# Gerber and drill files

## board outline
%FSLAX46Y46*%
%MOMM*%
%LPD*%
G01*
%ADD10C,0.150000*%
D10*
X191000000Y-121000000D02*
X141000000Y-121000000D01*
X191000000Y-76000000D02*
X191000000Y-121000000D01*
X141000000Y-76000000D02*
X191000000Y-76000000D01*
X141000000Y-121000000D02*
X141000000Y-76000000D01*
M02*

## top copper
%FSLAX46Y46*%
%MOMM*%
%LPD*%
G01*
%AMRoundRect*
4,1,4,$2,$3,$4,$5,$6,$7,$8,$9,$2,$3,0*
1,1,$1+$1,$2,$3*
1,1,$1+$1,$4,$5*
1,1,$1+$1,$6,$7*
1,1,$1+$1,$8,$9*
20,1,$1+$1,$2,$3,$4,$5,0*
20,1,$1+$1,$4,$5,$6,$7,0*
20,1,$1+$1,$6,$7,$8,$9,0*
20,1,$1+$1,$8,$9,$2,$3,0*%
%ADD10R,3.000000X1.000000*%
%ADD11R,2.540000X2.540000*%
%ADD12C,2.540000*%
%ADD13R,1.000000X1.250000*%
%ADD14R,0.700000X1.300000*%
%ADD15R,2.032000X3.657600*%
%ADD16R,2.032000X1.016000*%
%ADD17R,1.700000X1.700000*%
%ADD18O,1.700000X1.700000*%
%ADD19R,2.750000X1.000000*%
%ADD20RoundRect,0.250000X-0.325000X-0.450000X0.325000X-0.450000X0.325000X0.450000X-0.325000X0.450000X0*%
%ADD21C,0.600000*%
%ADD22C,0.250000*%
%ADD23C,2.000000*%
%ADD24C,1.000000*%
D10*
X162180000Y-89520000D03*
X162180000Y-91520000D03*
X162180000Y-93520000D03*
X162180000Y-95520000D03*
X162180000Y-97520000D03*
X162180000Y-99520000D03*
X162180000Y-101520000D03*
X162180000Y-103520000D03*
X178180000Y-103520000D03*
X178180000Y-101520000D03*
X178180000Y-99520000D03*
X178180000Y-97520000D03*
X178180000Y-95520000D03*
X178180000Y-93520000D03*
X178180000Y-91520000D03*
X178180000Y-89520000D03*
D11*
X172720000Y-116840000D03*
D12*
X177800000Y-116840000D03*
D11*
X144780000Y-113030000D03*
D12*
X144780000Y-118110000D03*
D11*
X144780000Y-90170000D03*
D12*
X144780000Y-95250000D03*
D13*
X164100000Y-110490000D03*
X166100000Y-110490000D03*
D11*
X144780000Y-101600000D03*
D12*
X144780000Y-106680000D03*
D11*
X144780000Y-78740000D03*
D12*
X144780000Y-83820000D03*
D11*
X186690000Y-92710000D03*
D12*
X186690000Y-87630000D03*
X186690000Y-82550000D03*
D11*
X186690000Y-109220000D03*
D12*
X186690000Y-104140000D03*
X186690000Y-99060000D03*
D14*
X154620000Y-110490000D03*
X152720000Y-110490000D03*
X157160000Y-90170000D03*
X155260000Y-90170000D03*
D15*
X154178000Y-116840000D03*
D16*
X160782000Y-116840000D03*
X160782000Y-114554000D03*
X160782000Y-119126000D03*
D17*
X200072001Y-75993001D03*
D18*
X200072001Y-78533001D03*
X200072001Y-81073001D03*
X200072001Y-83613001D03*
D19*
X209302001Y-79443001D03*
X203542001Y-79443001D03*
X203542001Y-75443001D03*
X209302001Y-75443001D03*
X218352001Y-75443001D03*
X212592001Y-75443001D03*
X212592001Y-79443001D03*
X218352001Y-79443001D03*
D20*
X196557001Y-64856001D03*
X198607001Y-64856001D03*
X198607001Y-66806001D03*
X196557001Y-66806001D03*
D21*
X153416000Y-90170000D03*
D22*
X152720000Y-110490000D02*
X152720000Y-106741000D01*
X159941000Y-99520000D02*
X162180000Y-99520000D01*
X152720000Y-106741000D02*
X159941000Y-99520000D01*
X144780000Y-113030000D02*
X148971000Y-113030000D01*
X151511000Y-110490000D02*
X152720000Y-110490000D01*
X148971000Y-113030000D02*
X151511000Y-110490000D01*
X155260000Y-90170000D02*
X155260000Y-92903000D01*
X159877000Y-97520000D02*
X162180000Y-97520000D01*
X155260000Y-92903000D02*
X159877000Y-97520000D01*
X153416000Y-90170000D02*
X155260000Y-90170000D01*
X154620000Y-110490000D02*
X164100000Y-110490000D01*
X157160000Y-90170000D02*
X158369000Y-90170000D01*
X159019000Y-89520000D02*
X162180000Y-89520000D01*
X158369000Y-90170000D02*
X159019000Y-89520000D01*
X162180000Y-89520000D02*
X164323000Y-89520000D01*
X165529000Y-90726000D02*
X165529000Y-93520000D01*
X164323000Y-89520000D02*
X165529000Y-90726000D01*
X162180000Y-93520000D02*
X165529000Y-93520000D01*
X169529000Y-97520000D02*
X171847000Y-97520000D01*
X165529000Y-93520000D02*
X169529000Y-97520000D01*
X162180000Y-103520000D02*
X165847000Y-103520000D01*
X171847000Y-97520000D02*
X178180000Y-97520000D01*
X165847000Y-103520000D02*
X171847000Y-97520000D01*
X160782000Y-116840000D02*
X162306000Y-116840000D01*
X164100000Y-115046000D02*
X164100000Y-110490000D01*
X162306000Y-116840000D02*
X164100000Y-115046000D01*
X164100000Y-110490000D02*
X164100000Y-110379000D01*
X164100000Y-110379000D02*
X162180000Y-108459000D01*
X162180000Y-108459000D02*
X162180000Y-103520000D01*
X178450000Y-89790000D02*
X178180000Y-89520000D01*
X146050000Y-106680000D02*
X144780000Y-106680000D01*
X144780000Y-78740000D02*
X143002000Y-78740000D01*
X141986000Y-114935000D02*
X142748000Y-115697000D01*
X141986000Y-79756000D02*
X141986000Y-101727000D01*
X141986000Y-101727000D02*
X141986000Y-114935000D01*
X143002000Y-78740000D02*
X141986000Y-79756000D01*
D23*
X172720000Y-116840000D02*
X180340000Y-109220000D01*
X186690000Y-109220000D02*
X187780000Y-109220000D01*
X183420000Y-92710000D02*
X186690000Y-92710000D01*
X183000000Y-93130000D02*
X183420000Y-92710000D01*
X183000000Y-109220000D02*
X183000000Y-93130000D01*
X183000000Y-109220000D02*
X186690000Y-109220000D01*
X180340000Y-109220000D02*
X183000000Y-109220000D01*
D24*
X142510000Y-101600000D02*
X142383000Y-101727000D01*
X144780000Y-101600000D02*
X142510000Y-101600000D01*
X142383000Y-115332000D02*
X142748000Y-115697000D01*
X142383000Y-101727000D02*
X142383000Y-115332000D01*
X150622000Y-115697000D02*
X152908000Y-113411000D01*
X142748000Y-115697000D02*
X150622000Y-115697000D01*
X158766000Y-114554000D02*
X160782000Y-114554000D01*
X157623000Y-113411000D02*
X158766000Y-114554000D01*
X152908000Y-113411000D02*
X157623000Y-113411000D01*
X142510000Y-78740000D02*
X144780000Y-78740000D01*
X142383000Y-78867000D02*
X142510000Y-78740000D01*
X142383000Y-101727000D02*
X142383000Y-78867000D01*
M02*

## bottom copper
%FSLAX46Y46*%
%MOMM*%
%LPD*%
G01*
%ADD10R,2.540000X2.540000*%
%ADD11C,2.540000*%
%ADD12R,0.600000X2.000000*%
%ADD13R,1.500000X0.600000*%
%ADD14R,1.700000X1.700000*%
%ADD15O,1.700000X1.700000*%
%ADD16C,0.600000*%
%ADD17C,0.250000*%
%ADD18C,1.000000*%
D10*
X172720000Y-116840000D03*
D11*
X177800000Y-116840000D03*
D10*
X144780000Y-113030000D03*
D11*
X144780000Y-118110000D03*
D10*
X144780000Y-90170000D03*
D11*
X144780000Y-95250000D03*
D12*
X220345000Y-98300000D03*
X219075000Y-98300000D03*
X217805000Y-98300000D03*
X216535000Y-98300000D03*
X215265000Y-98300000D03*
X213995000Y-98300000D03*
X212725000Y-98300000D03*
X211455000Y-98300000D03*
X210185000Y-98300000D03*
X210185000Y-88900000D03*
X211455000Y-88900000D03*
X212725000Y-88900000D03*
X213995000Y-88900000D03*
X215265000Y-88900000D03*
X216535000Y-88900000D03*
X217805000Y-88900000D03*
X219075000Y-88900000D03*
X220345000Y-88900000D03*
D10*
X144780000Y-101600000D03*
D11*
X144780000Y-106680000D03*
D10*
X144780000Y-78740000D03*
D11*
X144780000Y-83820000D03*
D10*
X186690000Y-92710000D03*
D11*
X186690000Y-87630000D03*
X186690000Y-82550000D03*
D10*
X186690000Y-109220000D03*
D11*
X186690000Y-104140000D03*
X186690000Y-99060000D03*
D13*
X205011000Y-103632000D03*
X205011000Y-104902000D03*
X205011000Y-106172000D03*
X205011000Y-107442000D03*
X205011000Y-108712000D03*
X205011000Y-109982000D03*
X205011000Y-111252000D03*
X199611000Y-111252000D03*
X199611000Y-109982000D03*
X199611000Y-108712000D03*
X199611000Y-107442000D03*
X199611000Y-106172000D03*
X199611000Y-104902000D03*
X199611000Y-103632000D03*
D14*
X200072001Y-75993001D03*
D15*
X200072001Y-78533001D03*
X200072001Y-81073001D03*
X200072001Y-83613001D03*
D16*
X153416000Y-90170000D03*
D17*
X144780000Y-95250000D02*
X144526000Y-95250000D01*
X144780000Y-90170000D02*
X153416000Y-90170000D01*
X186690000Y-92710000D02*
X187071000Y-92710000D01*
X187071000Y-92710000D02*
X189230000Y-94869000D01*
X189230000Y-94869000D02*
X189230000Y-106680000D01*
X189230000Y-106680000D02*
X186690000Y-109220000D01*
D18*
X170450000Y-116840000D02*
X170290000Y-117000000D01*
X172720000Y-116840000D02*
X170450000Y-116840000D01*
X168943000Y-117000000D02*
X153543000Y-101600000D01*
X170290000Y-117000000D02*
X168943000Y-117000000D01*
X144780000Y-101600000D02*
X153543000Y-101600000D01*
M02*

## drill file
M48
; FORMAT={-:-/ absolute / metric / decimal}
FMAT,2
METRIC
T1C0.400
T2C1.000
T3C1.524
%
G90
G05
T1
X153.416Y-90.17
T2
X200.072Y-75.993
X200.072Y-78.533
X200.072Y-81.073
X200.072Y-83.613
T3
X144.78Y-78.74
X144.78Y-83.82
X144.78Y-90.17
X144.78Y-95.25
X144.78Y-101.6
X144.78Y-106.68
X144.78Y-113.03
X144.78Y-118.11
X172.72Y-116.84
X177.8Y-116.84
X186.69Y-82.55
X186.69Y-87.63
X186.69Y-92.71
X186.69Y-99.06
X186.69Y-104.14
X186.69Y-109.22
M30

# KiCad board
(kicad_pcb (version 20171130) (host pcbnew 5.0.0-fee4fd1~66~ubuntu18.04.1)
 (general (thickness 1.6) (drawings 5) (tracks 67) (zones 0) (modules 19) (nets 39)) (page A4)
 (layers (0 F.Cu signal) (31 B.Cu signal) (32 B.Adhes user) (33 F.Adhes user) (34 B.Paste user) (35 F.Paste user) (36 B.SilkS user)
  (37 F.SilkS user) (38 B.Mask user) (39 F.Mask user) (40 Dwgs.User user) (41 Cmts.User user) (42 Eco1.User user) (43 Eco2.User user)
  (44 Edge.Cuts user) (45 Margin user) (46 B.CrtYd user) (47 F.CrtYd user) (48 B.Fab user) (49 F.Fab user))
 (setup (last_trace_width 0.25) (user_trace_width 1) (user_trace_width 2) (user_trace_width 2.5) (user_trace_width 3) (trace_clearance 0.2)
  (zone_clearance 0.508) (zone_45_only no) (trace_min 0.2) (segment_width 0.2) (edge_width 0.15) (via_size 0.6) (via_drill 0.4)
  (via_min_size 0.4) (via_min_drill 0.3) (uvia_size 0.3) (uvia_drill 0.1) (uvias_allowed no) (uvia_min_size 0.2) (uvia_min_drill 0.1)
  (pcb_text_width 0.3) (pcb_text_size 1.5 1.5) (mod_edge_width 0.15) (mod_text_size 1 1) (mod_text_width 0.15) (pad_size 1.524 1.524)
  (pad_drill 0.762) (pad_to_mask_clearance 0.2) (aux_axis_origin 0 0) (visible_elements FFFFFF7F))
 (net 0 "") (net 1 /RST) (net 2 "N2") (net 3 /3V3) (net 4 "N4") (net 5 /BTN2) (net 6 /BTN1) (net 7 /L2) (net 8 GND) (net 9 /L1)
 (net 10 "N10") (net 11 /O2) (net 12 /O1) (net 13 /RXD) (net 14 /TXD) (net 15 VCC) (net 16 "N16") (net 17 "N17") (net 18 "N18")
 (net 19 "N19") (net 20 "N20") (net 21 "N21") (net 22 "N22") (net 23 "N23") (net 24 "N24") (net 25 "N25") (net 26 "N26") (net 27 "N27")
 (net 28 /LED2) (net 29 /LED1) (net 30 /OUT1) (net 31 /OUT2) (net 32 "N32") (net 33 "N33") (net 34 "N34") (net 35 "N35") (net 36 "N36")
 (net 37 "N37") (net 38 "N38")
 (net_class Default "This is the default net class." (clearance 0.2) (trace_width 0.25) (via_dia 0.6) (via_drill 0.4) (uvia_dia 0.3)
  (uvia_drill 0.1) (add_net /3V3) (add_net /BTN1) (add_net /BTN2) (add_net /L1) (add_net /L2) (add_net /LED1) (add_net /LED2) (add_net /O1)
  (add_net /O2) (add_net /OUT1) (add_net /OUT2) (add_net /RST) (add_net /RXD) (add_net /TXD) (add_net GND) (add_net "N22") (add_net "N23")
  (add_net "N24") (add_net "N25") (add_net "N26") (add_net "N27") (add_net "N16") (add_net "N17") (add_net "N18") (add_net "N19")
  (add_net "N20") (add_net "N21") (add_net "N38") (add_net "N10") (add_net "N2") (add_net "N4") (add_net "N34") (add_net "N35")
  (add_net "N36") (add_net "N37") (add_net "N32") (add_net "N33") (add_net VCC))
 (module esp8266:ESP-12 (layer F.Cu) (at 170.18 96.52)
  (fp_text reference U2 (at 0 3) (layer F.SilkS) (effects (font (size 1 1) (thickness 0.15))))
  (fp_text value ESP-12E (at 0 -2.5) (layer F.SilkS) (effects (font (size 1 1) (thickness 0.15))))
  (pad 1 smd rect (at -8 -7) (size 3 1) (layers F.Cu F.Paste F.Mask) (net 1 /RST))
  (pad 2 smd rect (at -8 -5) (size 3 1) (layers F.Cu F.Paste F.Mask) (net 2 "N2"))
  (pad 3 smd rect (at -8 -3) (size 3 1) (layers F.Cu F.Paste F.Mask) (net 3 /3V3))
  (pad 4 smd rect (at -8 -1) (size 3 1) (layers F.Cu F.Paste F.Mask) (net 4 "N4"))
  (pad 5 smd rect (at -8 1) (size 3 1) (layers F.Cu F.Paste F.Mask) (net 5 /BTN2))
  (pad 6 smd rect (at -8 3) (size 3 1) (layers F.Cu F.Paste F.Mask) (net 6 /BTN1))
  (pad 7 smd rect (at -8 5) (size 3 1) (layers F.Cu F.Paste F.Mask) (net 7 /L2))
  (pad 8 smd rect (at -8 7) (size 3 1) (layers F.Cu F.Paste F.Mask) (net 3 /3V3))
  (pad 9 smd rect (at 8 7) (size 3 1) (layers F.Cu F.Paste F.Mask) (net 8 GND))
  (pad 10 smd rect (at 8 5) (size 3 1) (layers F.Cu F.Paste F.Mask) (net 8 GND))
  (pad 11 smd rect (at 8 3) (size 3 1) (layers F.Cu F.Paste F.Mask) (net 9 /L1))
  (pad 12 smd rect (at 8 1) (size 3 1) (layers F.Cu F.Paste F.Mask) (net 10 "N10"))
  (pad 13 smd rect (at 8 -1) (size 3 1) (layers F.Cu F.Paste F.Mask) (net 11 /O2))
  (pad 14 smd rect (at 8 -3) (size 3 1) (layers F.Cu F.Paste F.Mask) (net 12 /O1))
  (pad 15 smd rect (at 8 -5) (size 3 1) (layers F.Cu F.Paste F.Mask) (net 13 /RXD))
  (pad 16 smd rect (at 8 -7) (size 3 1) (layers F.Cu F.Paste F.Mask) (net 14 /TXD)))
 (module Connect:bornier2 (layer F.Cu) (at 175.26 116.84)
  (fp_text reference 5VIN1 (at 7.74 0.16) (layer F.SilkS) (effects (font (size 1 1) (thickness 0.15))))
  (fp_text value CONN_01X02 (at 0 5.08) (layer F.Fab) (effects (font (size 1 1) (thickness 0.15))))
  (pad 1 thru_hole rect (at -2.54 0) (size 2.54 2.54) (drill 1.524) (layers *.Cu *.Mask F.SilkS) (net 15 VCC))
  (pad 2 thru_hole circle (at 2.54 0) (size 2.54 2.54) (drill 1.524) (layers *.Cu *.Mask F.SilkS) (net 8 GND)))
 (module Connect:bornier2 (layer F.Cu) (at 144.78 115.57 270)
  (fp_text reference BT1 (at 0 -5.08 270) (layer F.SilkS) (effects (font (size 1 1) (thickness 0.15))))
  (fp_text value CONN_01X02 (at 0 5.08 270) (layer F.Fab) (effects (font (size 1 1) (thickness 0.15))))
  (pad 1 thru_hole rect (at -2.54 0 270) (size 2.54 2.54) (drill 1.524) (layers *.Cu *.Mask F.SilkS) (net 6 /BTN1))
  (pad 2 thru_hole circle (at 2.54 0 270) (size 2.54 2.54) (drill 1.524) (layers *.Cu *.Mask F.SilkS) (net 8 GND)))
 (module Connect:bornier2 (layer F.Cu) (at 144.78 92.71 270)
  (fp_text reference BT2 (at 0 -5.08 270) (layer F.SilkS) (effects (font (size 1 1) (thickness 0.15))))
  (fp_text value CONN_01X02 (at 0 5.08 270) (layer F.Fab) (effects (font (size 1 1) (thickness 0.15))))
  (pad 1 thru_hole rect (at -2.54 0 270) (size 2.54 2.54) (drill 1.524) (layers *.Cu *.Mask F.SilkS) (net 5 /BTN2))
  (pad 2 thru_hole circle (at 2.54 0 270) (size 2.54 2.54) (drill 1.524) (layers *.Cu *.Mask F.SilkS) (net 8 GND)))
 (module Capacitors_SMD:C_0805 (layer F.Cu) (at 165.1 110.49)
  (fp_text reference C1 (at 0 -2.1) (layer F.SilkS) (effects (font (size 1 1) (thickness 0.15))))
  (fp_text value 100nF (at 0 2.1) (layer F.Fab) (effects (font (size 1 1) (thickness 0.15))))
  (pad 1 smd rect (at -1 0) (size 1 1.25) (layers F.Cu F.Paste F.Mask) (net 3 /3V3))
  (pad 2 smd rect (at 1 0) (size 1 1.25) (layers F.Cu F.Paste F.Mask) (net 8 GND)))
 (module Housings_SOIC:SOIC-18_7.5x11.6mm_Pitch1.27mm (layer B.Cu) (at 215.265 93.6 90)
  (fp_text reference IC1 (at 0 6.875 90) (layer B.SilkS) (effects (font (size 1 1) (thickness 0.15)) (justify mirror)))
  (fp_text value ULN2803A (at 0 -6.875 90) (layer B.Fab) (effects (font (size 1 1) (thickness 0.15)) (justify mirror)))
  (pad 1 smd rect (at -4.7 5.08 90) (size 2 0.6) (layers B.Cu B.Paste B.Mask) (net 9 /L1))
  (pad 2 smd rect (at -4.7 3.81 90) (size 2 0.6) (layers B.Cu B.Paste B.Mask) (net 7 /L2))
  (pad 3 smd rect (at -4.7 2.54 90) (size 2 0.6) (layers B.Cu B.Paste B.Mask) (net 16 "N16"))
  (pad 4 smd rect (at -4.7 1.27 90) (size 2 0.6) (layers B.Cu B.Paste B.Mask) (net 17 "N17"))
  (pad 5 smd rect (at -4.7 0 90) (size 2 0.6) (layers B.Cu B.Paste B.Mask) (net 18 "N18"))
  (pad 6 smd rect (at -4.7 -1.27 90) (size 2 0.6) (layers B.Cu B.Paste B.Mask) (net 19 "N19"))
  (pad 7 smd rect (at -4.7 -2.54 90) (size 2 0.6) (layers B.Cu B.Paste B.Mask) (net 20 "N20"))
  (pad 8 smd rect (at -4.7 -3.81 90) (size 2 0.6) (layers B.Cu B.Paste B.Mask) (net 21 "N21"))
  (pad 9 smd rect (at -4.7 -5.08 90) (size 2 0.6) (layers B.Cu B.Paste B.Mask) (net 8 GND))
  (pad 10 smd rect (at 4.7 -5.08 90) (size 2 0.6) (layers B.Cu B.Paste B.Mask) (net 15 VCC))
  (pad 11 smd rect (at 4.7 -3.81 90) (size 2 0.6) (layers B.Cu B.Paste B.Mask) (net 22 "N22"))
  (pad 12 smd rect (at 4.7 -2.54 90) (size 2 0.6) (layers B.Cu B.Paste B.Mask) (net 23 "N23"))
  (pad 13 smd rect (at 4.7 -1.27 90) (size 2 0.6) (layers B.Cu B.Paste B.Mask) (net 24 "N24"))
  (pad 14 smd rect (at 4.7 0 90) (size 2 0.6) (layers B.Cu B.Paste B.Mask) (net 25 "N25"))
  (pad 15 smd rect (at 4.7 1.27 90) (size 2 0.6) (layers B.Cu B.Paste B.Mask) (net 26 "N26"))
  (pad 16 smd rect (at 4.7 2.54 90) (size 2 0.6) (layers B.Cu B.Paste B.Mask) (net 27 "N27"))
  (pad 17 smd rect (at 4.7 3.81 90) (size 2 0.6) (layers B.Cu B.Paste B.Mask) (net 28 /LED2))
  (pad 18 smd rect (at 4.7 5.08 90) (size 2 0.6) (layers B.Cu B.Paste B.Mask) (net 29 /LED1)))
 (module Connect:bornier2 (layer F.Cu) (at 144.78 104.14 270)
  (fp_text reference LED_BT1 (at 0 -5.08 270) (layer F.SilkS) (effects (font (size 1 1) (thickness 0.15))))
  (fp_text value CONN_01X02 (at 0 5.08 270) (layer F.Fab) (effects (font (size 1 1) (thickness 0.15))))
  (pad 1 thru_hole rect (at -2.54 0 270) (size 2.54 2.54) (drill 1.524) (layers *.Cu *.Mask F.SilkS) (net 15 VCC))
  (pad 2 thru_hole circle (at 2.54 0 270) (size 2.54 2.54) (drill 1.524) (layers *.Cu *.Mask F.SilkS) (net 29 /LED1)))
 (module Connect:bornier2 (layer F.Cu) (at 144.78 81.28 270)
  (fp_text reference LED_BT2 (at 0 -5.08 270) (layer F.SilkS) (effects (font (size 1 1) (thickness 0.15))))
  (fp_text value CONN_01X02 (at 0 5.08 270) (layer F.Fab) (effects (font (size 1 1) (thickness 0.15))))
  (pad 1 thru_hole rect (at -2.54 0 270) (size 2.54 2.54) (drill 1.524) (layers *.Cu *.Mask F.SilkS) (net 15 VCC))
  (pad 2 thru_hole circle (at 2.54 0 270) (size 2.54 2.54) (drill 1.524) (layers *.Cu *.Mask F.SilkS) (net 28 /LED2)))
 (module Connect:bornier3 (layer F.Cu) (at 186.69 87.63 90)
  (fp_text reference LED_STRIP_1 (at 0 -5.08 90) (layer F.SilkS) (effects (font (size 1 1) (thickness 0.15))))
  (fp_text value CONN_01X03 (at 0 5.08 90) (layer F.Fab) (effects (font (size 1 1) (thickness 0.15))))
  (pad 1 thru_hole rect (at -5.08 0 90) (size 2.54 2.54) (drill 1.524) (layers *.Cu *.Mask F.SilkS) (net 15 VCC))
  (pad 2 thru_hole circle (at 0 0 90) (size 2.54 2.54) (drill 1.524) (layers *.Cu *.Mask F.SilkS) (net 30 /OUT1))
  (pad 3 thru_hole circle (at 5.08 0 90) (size 2.54 2.54) (drill 1.524) (layers *.Cu *.Mask F.SilkS) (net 8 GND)))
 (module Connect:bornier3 (layer F.Cu) (at 186.69 104.14 90)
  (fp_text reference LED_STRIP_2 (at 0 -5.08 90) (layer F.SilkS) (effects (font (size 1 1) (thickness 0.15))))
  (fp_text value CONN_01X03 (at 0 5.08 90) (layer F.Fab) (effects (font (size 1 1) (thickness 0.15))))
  (pad 1 thru_hole rect (at -5.08 0 90) (size 2.54 2.54) (drill 1.524) (layers *.Cu *.Mask F.SilkS) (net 15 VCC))
  (pad 2 thru_hole circle (at 0 0 90) (size 2.54 2.54) (drill 1.524) (layers *.Cu *.Mask F.SilkS) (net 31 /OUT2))
  (pad 3 thru_hole circle (at 5.08 0 90) (size 2.54 2.54) (drill 1.524) (layers *.Cu *.Mask F.SilkS) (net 8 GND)))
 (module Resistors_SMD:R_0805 (layer F.Cu) (at 153.67 110.49 180)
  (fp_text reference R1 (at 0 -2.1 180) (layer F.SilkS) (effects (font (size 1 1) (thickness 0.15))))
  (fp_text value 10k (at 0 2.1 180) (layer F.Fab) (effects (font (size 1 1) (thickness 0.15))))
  (pad 1 smd rect (at -0.95 0 180) (size 0.7 1.3) (layers F.Cu F.Paste F.Mask) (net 3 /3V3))
  (pad 2 smd rect (at 0.95 0 180) (size 0.7 1.3) (layers F.Cu F.Paste F.Mask) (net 6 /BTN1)))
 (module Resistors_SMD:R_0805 (layer F.Cu) (at 156.21 90.17 180)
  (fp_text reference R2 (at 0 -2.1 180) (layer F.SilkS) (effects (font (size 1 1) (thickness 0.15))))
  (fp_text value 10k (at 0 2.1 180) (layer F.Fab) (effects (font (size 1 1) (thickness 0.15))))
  (pad 1 smd rect (at -0.95 0 180) (size 0.7 1.3) (layers F.Cu F.Paste F.Mask) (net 3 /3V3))
  (pad 2 smd rect (at 0.95 0 180) (size 0.7 1.3) (layers F.Cu F.Paste F.Mask) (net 5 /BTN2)))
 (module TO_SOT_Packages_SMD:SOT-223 (layer F.Cu) (at 157.48 116.84 90)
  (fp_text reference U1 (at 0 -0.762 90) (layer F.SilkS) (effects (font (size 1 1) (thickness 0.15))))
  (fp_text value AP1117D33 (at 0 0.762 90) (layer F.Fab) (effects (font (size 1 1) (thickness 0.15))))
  (pad 4 smd rect (at 0 -3.302 90) (size 3.6576 2.032) (layers F.Cu F.Paste F.Mask))
  (pad 2 smd rect (at 0 3.302 90) (size 1.016 2.032) (layers F.Cu F.Paste F.Mask) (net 3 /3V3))
  (pad 3 smd rect (at 2.286 3.302 90) (size 1.016 2.032) (layers F.Cu F.Paste F.Mask) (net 15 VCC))
  (pad 1 smd rect (at -2.286 3.302 90) (size 1.016 2.032) (layers F.Cu F.Paste F.Mask) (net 8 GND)))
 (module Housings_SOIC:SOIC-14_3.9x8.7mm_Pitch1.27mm (layer B.Cu) (at 202.311 107.442 180)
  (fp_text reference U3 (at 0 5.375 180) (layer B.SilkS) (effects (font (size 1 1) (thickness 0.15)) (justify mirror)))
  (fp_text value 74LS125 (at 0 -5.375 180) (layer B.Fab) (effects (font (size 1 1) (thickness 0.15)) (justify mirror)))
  (pad 1 smd rect (at -2.7 3.81 180) (size 1.5 0.6) (layers B.Cu B.Paste B.Mask) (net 8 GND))
  (pad 2 smd rect (at -2.7 2.54 180) (size 1.5 0.6) (layers B.Cu B.Paste B.Mask) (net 12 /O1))
  (pad 3 smd rect (at -2.7 1.27 180) (size 1.5 0.6) (layers B.Cu B.Paste B.Mask) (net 30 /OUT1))
  (pad 4 smd rect (at -2.7 0 180) (size 1.5 0.6) (layers B.Cu B.Paste B.Mask) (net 8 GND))
  (pad 5 smd rect (at -2.7 -1.27 180) (size 1.5 0.6) (layers B.Cu B.Paste B.Mask) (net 11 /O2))
  (pad 6 smd rect (at -2.7 -2.54 180) (size 1.5 0.6) (layers B.Cu B.Paste B.Mask) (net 31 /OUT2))
  (pad 7 smd rect (at -2.7 -3.81 180) (size 1.5 0.6) (layers B.Cu B.Paste B.Mask) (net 8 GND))
  (pad 8 smd rect (at 2.7 -3.81 180) (size 1.5 0.6) (layers B.Cu B.Paste B.Mask) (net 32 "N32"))
  (pad 9 smd rect (at 2.7 -2.54 180) (size 1.5 0.6) (layers B.Cu B.Paste B.Mask) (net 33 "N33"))
  (pad 10 smd rect (at 2.7 -1.27 180) (size 1.5 0.6) (layers B.Cu B.Paste B.Mask) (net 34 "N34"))
  (pad 11 smd rect (at 2.7 0 180) (size 1.5 0.6) (layers B.Cu B.Paste B.Mask) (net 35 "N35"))
  (pad 12 smd rect (at 2.7 1.27 180) (size 1.5 0.6) (layers B.Cu B.Paste B.Mask) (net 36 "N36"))
  (pad 13 smd rect (at 2.7 2.54 180) (size 1.5 0.6) (layers B.Cu B.Paste B.Mask) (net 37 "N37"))
  (pad 14 smd rect (at 2.7 3.81 180) (size 1.5 0.6) (layers B.Cu B.Paste B.Mask) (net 15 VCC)))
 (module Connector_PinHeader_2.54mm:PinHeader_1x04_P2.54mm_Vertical (layer F.Cu) (at 200.072001 75.993001)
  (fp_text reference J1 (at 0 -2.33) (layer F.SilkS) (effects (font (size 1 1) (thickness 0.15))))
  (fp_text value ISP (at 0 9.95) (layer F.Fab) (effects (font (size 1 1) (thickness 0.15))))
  (pad 1 thru_hole rect (at 0 0) (size 1.7 1.7) (drill 1) (layers *.Cu *.Mask) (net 3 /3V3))
  (pad 2 thru_hole oval (at 0 2.54) (size 1.7 1.7) (drill 1) (layers *.Cu *.Mask) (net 14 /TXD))
  (pad 3 thru_hole oval (at 0 5.08) (size 1.7 1.7) (drill 1) (layers *.Cu *.Mask) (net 13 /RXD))
  (pad 4 thru_hole oval (at 0 7.62) (size 1.7 1.7) (drill 1) (layers *.Cu *.Mask) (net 8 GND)))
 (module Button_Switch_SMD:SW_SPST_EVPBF (layer F.Cu) (at 206.422001 77.443001)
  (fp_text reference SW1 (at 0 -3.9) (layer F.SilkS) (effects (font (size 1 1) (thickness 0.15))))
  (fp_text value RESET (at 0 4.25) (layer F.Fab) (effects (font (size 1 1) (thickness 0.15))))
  (pad 2 smd rect (at 2.88 2) (size 2.75 1) (layers F.Cu F.Paste F.Mask) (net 8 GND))
  (pad 2 smd rect (at -2.88 2) (size 2.75 1) (layers F.Cu F.Paste F.Mask) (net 8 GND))
  (pad 1 smd rect (at -2.88 -2) (size 2.75 1) (layers F.Cu F.Paste F.Mask) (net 1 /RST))
  (pad 1 smd rect (at 2.88 -2) (size 2.75 1) (layers F.Cu F.Paste F.Mask) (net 1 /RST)))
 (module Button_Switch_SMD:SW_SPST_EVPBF (layer F.Cu) (at 215.472001 77.443001)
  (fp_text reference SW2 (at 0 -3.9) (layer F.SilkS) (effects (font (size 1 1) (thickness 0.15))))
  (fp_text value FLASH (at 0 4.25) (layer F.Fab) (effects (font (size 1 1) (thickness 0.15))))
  (pad 1 smd rect (at 2.88 -2) (size 2.75 1) (layers F.Cu F.Paste F.Mask) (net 10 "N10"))
  (pad 1 smd rect (at -2.88 -2) (size 2.75 1) (layers F.Cu F.Paste F.Mask) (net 10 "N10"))
  (pad 2 smd rect (at -2.88 2) (size 2.75 1) (layers F.Cu F.Paste F.Mask) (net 8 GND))
  (pad 2 smd rect (at 2.88 2) (size 2.75 1) (layers F.Cu F.Paste F.Mask) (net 8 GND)))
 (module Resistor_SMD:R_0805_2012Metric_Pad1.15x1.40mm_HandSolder (layer F.Cu) (at 197.582001 64.856001)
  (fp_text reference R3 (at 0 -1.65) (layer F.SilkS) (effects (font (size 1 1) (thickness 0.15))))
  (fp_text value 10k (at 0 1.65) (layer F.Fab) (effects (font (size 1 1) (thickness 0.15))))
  (pad 1 smd roundrect (at -1.025 0) (size 1.15 1.4) (layers F.Cu F.Paste F.Mask) (roundrect_rratio 0.217391) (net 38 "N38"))
  (pad 2 smd roundrect (at 1.025 0) (size 1.15 1.4) (layers F.Cu F.Paste F.Mask) (roundrect_rratio 0.217391) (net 1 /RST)))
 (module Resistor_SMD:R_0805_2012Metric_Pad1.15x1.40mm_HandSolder (layer F.Cu) (at 197.582001 66.806001)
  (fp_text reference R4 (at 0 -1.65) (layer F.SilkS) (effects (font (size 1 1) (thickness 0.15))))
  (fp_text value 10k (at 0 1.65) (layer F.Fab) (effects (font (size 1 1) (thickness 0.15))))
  (pad 2 smd roundrect (at 1.025 0) (size 1.15 1.4) (layers F.Cu F.Paste F.Mask) (roundrect_rratio 0.217391) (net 10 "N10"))
  (pad 1 smd roundrect (at -1.025 0) (size 1.15 1.4) (layers F.Cu F.Paste F.Mask) (roundrect_rratio 0.217391) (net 3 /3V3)))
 (gr_line (start 191 121) (end 141 121) (angle 90) (layer Edge.Cuts) (width 0.15))
 (gr_line (start 191 76) (end 191 121) (angle 90) (layer Edge.Cuts) (width 0.15))
 (gr_line (start 141 76) (end 191 76) (angle 90) (layer Edge.Cuts) (width 0.15))
 (gr_line (start 141 121) (end 141 76) (angle 90) (layer Edge.Cuts) (width 0.15))
 (segment (start 144.78 95.25) (end 144.526 95.25) (width 0.25) (layer B.Cu) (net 8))
 (segment (start 152.72 110.49) (end 152.72 106.741) (width 0.25) (layer F.Cu) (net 6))
 (segment (start 159.941 99.52) (end 162.18 99.52) (width 0.25) (layer F.Cu) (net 6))
 (segment (start 152.72 106.741) (end 159.941 99.52) (width 0.25) (layer F.Cu) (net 6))
 (segment (start 144.78 113.03) (end 148.971 113.03) (width 0.25) (layer F.Cu) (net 6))
 (segment (start 151.511 110.49) (end 152.72 110.49) (width 0.25) (layer F.Cu) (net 6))
 (segment (start 148.971 113.03) (end 151.511 110.49) (width 0.25) (layer F.Cu) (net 6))
 (segment (start 155.26 90.17) (end 155.26 92.903) (width 0.25) (layer F.Cu) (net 5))
 (segment (start 159.877 97.52) (end 162.18 97.52) (width 0.25) (layer F.Cu) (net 5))
 (segment (start 155.26 92.903) (end 159.877 97.52) (width 0.25) (layer F.Cu) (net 5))
 (segment (start 144.78 90.17) (end 153.416 90.17) (width 0.25) (layer B.Cu) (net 5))
 (segment (start 153.416 90.17) (end 155.26 90.17) (width 0.25) (layer F.Cu) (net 5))
 (via (at 153.416 90.17) (size 0.6) (drill 0.4) (layers F.Cu B.Cu) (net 5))
 (segment (start 154.62 110.49) (end 164.1 110.49) (width 0.25) (layer F.Cu) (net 3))
 (segment (start 157.16 90.17) (end 158.369 90.17) (width 0.25) (layer F.Cu) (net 3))
 (segment (start 159.019 89.52) (end 162.18 89.52) (width 0.25) (layer F.Cu) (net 3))
 (segment (start 158.369 90.17) (end 159.019 89.52) (width 0.25) (layer F.Cu) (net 3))
 (segment (start 162.18 89.52) (end 164.323 89.52) (width 0.25) (layer F.Cu) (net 3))
 (segment (start 165.529 90.726) (end 165.529 93.52) (width 0.25) (layer F.Cu) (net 3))
 (segment (start 164.323 89.52) (end 165.529 90.726) (width 0.25) (layer F.Cu) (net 3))
 (segment (start 162.18 93.52) (end 165.529 93.52) (width 0.25) (layer F.Cu) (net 3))
 (segment (start 169.529 97.52) (end 171.847 97.52) (width 0.25) (layer F.Cu) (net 3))
 (segment (start 165.529 93.52) (end 169.529 97.52) (width 0.25) (layer F.Cu) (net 3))
 (segment (start 162.18 103.52) (end 165.847 103.52) (width 0.25) (layer F.Cu) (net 3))
 (segment (start 171.847 97.52) (end 178.18 97.52) (width 0.25) (layer F.Cu) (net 3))
 (segment (start 165.847 103.52) (end 171.847 97.52) (width 0.25) (layer F.Cu) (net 3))
 (segment (start 160.782 116.84) (end 162.306 116.84) (width 0.25) (layer F.Cu) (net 3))
 (segment (start 164.1 115.046) (end 164.1 110.49) (width 0.25) (layer F.Cu) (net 3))
 (segment (start 162.306 116.84) (end 164.1 115.046) (width 0.25) (layer F.Cu) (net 3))
 (segment (start 164.1 110.49) (end 164.1 110.379) (width 0.25) (layer F.Cu) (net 3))
 (segment (start 164.1 110.379) (end 162.18 108.459) (width 0.25) (layer F.Cu) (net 3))
 (segment (start 162.18 108.459) (end 162.18 103.52) (width 0.25) (layer F.Cu) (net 3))
 (segment (start 178.45 89.79) (end 178.18 89.52) (width 0.25) (layer F.Cu) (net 14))
 (segment (start 146.05 106.68) (end 144.78 106.68) (width 0.25) (layer F.Cu) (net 29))
 (segment (start 186.69 92.71) (end 187.071 92.71) (width 0.25) (layer B.Cu) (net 15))
 (segment (start 187.071 92.71) (end 189.23 94.869) (width 0.25) (layer B.Cu) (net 15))
 (segment (start 189.23 94.869) (end 189.23 106.68) (width 0.25) (layer B.Cu) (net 15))
 (segment (start 189.23 106.68) (end 186.69 109.22) (width 0.25) (layer B.Cu) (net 15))
 (segment (start 144.78 78.74) (end 143.002 78.74) (width 0.25) (layer F.Cu) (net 15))
 (segment (start 141.986 114.935) (end 142.748 115.697) (width 0.25) (layer F.Cu) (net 15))
 (segment (start 141.986 79.756) (end 141.986 101.727) (width 0.25) (layer F.Cu) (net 15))
 (segment (start 141.986 101.727) (end 141.986 114.935) (width 0.25) (layer F.Cu) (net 15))
 (segment (start 143.002 78.74) (end 141.986 79.756) (width 0.25) (layer F.Cu) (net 15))
 (segment (start 172.72 116.84) (end 180.34 109.22) (width 2) (layer F.Cu) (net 15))
 (segment (start 186.69 109.22) (end 187.78 109.22) (width 2) (layer F.Cu) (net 15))
 (segment (start 183.42 92.71) (end 186.69 92.71) (width 2) (layer F.Cu) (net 15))
 (segment (start 183 93.13) (end 183.42 92.71) (width 2) (layer F.Cu) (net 15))
 (segment (start 183 109.22) (end 183 93.13) (width 2) (layer F.Cu) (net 15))
 (segment (start 183 109.22) (end 186.69 109.22) (width 2) (layer F.Cu) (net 15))
 (segment (start 180.34 109.22) (end 183 109.22) (width 2) (layer F.Cu) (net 15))
 (segment (start 170.45 116.84) (end 170.29 117) (width 1) (layer B.Cu) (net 15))
 (segment (start 172.72 116.84) (end 170.45 116.84) (width 1) (layer B.Cu) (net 15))
 (segment (start 168.943 117) (end 153.543 101.6) (width 1) (layer B.Cu) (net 15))
 (segment (start 170.29 117) (end 168.943 117) (width 1) (layer B.Cu) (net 15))
 (segment (start 144.78 101.6) (end 153.543 101.6) (width 1) (layer B.Cu) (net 15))
 (segment (start 142.51 101.6) (end 142.383 101.727) (width 1) (layer F.Cu) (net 15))
 (segment (start 144.78 101.6) (end 142.51 101.6) (width 1) (layer F.Cu) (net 15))
 (segment (start 142.383 115.332) (end 142.748 115.697) (width 1) (layer F.Cu) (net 15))
 (segment (start 142.383 101.727) (end 142.383 115.332) (width 1) (layer F.Cu) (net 15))
 (segment (start 150.622 115.697) (end 152.908 113.411) (width 1) (layer F.Cu) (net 15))
 (segment (start 142.748 115.697) (end 150.622 115.697) (width 1) (layer F.Cu) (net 15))
 (segment (start 158.766 114.554) (end 160.782 114.554) (width 1) (layer F.Cu) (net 15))
 (segment (start 157.623 113.411) (end 158.766 114.554) (width 1) (layer F.Cu) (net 15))
 (segment (start 152.908 113.411) (end 157.623 113.411) (width 1) (layer F.Cu) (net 15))
 (segment (start 142.51 78.74) (end 144.78 78.74) (width 1) (layer F.Cu) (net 15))
 (segment (start 142.383 78.867) (end 142.51 78.74) (width 1) (layer F.Cu) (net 15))
 (segment (start 142.383 101.727) (end 142.383 78.867) (width 1) (layer F.Cu) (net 15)))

